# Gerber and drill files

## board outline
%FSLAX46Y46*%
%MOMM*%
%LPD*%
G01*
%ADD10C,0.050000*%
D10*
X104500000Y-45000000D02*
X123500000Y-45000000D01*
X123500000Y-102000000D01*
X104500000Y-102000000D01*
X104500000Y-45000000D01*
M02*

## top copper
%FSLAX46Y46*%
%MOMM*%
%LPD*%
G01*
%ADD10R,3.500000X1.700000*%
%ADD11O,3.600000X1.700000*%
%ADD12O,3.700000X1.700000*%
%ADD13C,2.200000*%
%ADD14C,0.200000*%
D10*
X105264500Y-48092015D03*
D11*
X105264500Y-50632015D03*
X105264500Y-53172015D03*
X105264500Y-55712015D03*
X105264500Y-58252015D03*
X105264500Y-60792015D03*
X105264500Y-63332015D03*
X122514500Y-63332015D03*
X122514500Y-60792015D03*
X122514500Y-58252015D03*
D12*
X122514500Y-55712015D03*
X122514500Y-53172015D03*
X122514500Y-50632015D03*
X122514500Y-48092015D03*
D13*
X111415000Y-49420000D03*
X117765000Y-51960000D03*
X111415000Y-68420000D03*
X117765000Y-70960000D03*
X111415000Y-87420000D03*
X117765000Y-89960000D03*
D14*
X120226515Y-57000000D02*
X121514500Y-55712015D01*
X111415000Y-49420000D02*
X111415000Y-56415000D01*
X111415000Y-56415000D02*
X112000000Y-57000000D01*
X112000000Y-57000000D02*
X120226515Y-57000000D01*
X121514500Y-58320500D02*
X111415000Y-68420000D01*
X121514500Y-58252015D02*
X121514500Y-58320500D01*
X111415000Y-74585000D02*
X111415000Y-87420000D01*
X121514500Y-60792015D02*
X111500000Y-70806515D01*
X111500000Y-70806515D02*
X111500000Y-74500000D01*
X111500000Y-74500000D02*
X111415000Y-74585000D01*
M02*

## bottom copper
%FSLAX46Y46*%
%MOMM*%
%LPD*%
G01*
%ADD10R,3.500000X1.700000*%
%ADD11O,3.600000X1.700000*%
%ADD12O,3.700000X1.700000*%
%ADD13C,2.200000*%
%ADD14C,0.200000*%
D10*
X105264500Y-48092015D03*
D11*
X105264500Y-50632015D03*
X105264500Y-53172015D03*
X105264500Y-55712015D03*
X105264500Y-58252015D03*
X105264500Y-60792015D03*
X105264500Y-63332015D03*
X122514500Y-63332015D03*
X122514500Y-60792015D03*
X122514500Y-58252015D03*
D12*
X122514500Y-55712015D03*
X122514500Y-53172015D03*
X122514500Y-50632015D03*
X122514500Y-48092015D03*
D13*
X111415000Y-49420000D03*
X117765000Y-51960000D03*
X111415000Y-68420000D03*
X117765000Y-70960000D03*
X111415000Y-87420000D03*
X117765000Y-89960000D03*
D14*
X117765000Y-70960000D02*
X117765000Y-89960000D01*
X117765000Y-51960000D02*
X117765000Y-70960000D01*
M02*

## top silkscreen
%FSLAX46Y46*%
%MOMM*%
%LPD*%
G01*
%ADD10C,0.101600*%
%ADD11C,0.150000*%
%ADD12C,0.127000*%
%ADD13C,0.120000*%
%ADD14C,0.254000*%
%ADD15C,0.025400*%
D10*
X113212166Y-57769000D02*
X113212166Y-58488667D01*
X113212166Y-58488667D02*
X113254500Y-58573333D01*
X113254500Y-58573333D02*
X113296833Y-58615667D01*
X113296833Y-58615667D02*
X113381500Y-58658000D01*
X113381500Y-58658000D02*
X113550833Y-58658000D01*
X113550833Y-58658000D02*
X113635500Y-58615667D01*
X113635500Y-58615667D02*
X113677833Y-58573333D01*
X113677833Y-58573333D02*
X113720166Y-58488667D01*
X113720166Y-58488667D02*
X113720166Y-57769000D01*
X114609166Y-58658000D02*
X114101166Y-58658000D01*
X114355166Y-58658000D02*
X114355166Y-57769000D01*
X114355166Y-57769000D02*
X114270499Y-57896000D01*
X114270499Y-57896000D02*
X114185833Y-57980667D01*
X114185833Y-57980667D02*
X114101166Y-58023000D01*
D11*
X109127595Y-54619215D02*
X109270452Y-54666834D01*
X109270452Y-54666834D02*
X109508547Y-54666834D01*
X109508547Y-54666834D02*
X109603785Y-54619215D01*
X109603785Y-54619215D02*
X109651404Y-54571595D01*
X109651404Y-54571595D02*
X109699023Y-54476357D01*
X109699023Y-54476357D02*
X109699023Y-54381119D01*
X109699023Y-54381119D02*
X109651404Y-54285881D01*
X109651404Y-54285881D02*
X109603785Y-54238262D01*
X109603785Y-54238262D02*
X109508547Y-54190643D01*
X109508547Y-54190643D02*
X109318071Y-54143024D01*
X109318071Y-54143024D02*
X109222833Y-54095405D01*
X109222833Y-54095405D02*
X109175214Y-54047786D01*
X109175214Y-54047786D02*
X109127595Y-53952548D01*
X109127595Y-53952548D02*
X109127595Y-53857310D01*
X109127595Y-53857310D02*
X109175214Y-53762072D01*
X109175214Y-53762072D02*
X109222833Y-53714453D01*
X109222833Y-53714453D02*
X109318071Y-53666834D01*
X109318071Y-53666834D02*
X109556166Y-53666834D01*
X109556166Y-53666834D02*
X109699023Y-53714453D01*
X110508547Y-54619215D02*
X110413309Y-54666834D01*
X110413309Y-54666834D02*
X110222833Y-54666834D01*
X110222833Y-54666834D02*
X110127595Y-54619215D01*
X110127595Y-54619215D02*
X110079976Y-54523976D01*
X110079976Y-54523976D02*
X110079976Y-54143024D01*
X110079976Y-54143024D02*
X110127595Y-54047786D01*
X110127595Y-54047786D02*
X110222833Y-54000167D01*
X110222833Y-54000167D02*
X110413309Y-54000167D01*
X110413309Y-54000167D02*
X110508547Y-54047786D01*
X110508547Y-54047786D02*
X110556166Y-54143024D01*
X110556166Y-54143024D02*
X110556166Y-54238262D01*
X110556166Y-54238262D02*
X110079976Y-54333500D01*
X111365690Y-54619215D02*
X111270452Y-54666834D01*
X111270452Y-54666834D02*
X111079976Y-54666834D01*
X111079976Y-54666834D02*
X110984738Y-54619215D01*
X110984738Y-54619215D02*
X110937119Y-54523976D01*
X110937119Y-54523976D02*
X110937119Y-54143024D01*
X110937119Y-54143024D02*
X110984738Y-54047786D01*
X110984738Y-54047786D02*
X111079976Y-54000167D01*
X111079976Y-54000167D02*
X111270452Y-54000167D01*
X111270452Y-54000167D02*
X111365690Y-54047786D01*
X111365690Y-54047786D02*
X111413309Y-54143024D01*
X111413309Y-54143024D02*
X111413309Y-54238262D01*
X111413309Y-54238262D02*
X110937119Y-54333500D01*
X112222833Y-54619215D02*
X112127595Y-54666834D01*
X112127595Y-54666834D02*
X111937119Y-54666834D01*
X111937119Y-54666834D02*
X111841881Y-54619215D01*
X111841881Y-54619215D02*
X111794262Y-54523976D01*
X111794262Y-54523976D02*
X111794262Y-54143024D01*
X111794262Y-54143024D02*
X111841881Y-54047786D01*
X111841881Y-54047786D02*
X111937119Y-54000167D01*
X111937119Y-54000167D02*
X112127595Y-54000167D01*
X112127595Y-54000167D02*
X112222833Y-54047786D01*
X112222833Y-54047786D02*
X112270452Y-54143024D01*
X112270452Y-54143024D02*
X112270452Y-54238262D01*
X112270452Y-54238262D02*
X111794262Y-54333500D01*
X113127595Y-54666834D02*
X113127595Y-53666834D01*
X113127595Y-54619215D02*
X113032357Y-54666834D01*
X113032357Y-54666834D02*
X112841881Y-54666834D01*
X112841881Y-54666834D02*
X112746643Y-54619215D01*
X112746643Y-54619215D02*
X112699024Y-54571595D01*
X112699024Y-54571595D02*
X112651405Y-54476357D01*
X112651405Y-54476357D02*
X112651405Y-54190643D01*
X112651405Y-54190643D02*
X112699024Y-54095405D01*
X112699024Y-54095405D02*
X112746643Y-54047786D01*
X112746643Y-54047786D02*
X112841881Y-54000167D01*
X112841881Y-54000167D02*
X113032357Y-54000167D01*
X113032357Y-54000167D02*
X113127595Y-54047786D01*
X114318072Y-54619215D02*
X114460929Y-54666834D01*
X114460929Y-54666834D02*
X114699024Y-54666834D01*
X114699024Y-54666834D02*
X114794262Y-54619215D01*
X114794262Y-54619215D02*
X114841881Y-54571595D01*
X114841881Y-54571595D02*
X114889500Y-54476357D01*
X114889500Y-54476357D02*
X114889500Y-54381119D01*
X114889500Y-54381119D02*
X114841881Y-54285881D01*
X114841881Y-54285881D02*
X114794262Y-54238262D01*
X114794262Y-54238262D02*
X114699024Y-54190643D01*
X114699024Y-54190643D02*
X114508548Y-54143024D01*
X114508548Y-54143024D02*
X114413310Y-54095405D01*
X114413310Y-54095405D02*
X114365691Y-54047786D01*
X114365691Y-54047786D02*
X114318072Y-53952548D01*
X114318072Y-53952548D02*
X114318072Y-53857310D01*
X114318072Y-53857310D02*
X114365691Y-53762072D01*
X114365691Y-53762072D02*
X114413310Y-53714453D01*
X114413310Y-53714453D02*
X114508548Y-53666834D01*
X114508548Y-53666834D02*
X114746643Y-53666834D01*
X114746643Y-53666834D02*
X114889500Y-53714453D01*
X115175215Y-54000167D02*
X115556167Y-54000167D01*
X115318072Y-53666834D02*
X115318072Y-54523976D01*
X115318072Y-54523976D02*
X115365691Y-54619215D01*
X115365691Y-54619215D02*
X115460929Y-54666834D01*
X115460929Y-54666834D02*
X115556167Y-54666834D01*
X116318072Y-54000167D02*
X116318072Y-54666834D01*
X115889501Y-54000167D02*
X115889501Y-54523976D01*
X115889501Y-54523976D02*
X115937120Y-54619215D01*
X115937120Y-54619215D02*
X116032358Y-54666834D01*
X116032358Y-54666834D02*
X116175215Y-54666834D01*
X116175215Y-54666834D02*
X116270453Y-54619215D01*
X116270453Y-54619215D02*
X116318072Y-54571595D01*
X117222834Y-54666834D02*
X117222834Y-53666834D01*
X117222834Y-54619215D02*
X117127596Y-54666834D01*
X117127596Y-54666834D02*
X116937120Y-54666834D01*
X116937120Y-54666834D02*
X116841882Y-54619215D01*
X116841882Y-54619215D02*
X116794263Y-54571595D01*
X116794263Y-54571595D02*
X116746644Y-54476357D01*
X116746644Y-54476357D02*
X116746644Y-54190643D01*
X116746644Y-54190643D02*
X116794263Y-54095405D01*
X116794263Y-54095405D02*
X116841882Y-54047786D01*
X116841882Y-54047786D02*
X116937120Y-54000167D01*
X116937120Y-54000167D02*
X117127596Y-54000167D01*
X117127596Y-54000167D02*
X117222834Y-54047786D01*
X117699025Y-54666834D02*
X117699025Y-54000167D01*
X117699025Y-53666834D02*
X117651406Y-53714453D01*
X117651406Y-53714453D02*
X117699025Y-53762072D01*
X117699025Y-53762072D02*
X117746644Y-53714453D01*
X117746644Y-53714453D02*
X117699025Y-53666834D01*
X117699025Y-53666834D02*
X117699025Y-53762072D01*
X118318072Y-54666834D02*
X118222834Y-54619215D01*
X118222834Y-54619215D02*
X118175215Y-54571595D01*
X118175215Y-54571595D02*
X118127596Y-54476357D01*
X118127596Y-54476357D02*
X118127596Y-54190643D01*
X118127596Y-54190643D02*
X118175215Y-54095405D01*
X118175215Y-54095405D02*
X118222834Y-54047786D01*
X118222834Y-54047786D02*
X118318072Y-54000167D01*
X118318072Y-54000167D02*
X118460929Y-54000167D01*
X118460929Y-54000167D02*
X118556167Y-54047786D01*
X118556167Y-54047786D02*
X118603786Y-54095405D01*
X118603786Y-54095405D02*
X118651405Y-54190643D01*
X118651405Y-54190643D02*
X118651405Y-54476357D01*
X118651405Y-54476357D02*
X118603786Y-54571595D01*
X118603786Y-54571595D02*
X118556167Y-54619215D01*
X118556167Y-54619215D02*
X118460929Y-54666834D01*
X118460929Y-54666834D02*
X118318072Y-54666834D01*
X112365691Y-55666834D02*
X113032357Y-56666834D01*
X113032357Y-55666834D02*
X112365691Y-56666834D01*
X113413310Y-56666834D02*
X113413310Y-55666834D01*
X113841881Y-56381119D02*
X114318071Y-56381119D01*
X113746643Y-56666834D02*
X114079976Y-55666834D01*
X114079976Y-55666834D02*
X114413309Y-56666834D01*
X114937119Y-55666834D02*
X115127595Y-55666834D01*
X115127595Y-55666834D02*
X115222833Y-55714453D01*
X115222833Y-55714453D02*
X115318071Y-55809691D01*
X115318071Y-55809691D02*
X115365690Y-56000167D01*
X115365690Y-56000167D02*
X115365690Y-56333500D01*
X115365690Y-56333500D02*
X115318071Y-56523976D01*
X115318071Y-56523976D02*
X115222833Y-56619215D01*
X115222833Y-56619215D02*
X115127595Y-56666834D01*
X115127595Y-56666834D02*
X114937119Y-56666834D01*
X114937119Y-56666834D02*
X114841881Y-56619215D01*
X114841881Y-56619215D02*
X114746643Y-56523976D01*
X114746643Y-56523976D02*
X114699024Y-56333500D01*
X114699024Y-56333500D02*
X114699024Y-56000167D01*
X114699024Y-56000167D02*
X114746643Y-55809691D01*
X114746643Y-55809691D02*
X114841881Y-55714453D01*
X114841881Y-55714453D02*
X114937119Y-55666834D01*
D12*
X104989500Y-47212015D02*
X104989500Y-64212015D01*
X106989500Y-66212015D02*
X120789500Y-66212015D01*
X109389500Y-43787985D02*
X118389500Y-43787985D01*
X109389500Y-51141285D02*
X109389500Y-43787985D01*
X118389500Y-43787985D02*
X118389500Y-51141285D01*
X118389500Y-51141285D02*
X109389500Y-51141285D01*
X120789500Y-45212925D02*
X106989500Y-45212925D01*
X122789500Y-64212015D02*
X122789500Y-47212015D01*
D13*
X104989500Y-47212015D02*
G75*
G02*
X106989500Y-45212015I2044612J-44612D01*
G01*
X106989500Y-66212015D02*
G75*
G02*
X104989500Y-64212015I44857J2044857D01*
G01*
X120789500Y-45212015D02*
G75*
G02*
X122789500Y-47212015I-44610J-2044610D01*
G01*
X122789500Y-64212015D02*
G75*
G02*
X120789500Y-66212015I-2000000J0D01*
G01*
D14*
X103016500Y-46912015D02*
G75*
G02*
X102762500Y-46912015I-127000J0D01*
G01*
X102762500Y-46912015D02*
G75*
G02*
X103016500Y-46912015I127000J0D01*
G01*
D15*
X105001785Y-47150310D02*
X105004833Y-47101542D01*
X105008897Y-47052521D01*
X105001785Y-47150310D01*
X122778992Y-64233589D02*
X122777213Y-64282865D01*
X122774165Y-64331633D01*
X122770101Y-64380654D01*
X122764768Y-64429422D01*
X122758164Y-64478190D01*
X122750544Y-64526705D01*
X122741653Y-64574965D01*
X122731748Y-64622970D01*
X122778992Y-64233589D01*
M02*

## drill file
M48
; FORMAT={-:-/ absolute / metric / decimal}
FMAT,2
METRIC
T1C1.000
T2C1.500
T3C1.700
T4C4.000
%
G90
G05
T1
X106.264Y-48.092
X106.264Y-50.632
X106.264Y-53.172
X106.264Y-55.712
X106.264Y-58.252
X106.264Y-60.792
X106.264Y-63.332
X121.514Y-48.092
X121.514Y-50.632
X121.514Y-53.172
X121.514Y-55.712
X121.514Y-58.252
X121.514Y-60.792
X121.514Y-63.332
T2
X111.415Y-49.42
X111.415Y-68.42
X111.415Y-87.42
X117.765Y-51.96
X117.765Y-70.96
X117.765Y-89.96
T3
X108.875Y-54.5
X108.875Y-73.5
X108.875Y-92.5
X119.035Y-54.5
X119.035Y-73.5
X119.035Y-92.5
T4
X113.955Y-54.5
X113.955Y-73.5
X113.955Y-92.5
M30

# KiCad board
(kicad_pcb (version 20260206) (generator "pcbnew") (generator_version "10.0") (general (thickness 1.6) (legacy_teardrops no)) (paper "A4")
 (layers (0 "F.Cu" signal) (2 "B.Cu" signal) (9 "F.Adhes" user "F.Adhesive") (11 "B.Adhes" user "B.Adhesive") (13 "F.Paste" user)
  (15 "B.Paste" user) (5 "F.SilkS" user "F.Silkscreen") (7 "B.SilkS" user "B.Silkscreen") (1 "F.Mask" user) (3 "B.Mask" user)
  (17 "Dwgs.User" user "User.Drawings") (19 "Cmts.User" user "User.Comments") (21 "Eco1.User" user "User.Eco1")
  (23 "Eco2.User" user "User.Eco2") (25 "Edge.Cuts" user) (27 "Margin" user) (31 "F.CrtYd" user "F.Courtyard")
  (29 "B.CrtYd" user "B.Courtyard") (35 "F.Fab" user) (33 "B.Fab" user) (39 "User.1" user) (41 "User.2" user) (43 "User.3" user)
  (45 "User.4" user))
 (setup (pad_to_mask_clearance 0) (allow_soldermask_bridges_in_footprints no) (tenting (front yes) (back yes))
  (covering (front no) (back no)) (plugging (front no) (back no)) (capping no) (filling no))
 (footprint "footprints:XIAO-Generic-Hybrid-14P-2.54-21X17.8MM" (layer "F.Cu") (at 113.8895 55.712015)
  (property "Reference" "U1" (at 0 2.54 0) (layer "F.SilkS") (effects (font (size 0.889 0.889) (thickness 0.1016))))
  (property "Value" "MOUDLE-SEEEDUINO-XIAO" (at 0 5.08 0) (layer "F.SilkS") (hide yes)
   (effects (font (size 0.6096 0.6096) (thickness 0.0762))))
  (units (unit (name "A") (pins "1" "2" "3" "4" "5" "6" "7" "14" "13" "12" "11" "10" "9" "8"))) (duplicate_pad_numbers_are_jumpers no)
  (fp_line (start -8.9 -8.5) (end -8.9 8.5) (stroke (width 0.127) (type solid)) (layer "F.SilkS"))
  (fp_line (start -6.9 10.5) (end 6.9 10.5) (stroke (width 0.127) (type solid)) (layer "F.SilkS"))
  (fp_line (start -4.5 -11.92403) (end 4.5 -11.92403) (stroke (width 0.127) (type solid)) (layer "F.SilkS"))
  (fp_line (start -4.5 -4.57073) (end -4.5 -11.92403) (stroke (width 0.127) (type solid)) (layer "F.SilkS"))
  (fp_line (start 4.5 -11.92403) (end 4.5 -4.57073) (stroke (width 0.127) (type solid)) (layer "F.SilkS"))
  (fp_line (start 4.5 -4.57073) (end -4.5 -4.57073) (stroke (width 0.127) (type solid)) (layer "F.SilkS"))
  (fp_line (start 6.9 -10.49909) (end -6.9 -10.49909) (stroke (width 0.127) (type solid)) (layer "F.SilkS"))
  (fp_line (start 8.9 8.5) (end 8.9 -8.5) (stroke (width 0.127) (type solid)) (layer "F.SilkS"))
  (fp_arc (start -8.9 -8.5) (mid -8.301491 -9.901491) (end -6.9 -10.5) (stroke (width 0.12) (type solid)) (layer "F.SilkS"))
  (fp_arc (start -6.9 10.5) (mid -8.301423 9.901423) (end -8.9 8.5) (stroke (width 0.12) (type solid)) (layer "F.SilkS"))
  (fp_arc (start 6.9 -10.5) (mid 8.301491 -9.901491) (end 8.9 -8.5) (stroke (width 0.12) (type solid)) (layer "F.SilkS"))
  (fp_arc (start 8.9 8.5) (mid 8.314214 9.914214) (end 6.9 10.5) (stroke (width 0.12) (type solid)) (layer "F.SilkS"))
  (fp_circle (center -11 -8.8) (end -11 -9.054) (stroke (width 0) (type solid)) (fill yes) (layer "F.SilkS"))
  (fp_poly
   (pts (xy -8.887715 -8.561705) (xy -8.884667 -8.610473) (xy -8.880603 -8.659494)) (stroke (width 0.0254) (type solid)) (fill no)
   (layer "F.SilkS"))
  (fp_poly
   (pts (xy 8.889492 8.521574) (xy 8.887713 8.57085) (xy 8.884665 8.619618) (xy 8.880601 8.668639) (xy 8.875268 8.717407)
    (xy 8.868664 8.766175) (xy 8.861044 8.81469) (xy 8.852153 8.86295) (xy 8.842248 8.910955))
   (stroke (width 0.0254) (type solid)) (fill no) (layer "F.SilkS"))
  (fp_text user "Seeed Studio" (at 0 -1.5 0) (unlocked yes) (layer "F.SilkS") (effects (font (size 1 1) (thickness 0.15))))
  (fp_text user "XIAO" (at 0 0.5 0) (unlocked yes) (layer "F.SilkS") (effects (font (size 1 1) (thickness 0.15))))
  (pad "1" thru_hole rect (at -7.625 -7.62) (size 3.5 1.7) (drill 1 (offset -1 0)) (layers "*.Cu" "*.Mask") (remove_unused_layers no)
   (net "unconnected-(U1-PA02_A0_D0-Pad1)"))
  (pad "2" thru_hole oval (at -7.625 -5.08) (size 3.6 1.7) (drill 1 (offset -1 0)) (layers "*.Cu" "*.Mask") (remove_unused_layers no)
   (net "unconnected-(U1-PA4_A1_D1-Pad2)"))
  (pad "3" thru_hole oval (at -7.625 -2.54) (size 3.6 1.7) (drill 1 (offset -1 0)) (layers "*.Cu" "*.Mask") (remove_unused_layers no)
   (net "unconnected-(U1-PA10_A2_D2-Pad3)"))
  (pad "4" thru_hole oval (at -7.625 0) (size 3.6 1.7) (drill 1 (offset -1 0)) (layers "*.Cu" "*.Mask") (remove_unused_layers no)
   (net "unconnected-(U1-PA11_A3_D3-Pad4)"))
  (pad "5" thru_hole oval (at -7.625 2.54) (size 3.6 1.7) (drill 1 (offset -1 0)) (layers "*.Cu" "*.Mask") (remove_unused_layers no)
   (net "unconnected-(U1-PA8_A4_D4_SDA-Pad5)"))
  (pad "6" thru_hole oval (at -7.625 5.08 180) (size 3.6 1.7) (drill 1 (offset 1 0)) (layers "*.Cu" "*.Mask") (remove_unused_layers no)
   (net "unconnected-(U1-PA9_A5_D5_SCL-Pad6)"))
  (pad "7" thru_hole oval (at -7.625 7.62) (size 3.6 1.7) (drill 1 (offset -1 0)) (layers "*.Cu" "*.Mask") (remove_unused_layers no)
   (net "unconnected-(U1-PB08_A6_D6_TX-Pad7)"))
  (pad "8" thru_hole oval (at 7.625 7.62) (size 3.6 1.7) (drill 1 (offset 1 0)) (layers "*.Cu" "*.Mask") (remove_unused_layers no)
   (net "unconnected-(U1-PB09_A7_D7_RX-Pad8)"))
  (pad "9" thru_hole oval (at 7.625 5.08) (size 3.6 1.7) (drill 1 (offset 1 0)) (layers "*.Cu" "*.Mask") (remove_unused_layers no)
   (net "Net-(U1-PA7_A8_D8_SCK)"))
  (pad "10" thru_hole oval (at 7.625 2.54) (size 3.6 1.7) (drill 1 (offset 1 0)) (layers "*.Cu" "*.Mask") (remove_unused_layers no)
   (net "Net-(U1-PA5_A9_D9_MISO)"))
  (pad "11" thru_hole oval (at 7.625 0) (size 3.7 1.7) (drill 1 (offset 1 0)) (layers "*.Cu" "*.Mask") (remove_unused_layers no)
   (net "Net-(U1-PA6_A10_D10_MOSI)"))
  (pad "12" thru_hole oval (at 7.625 -2.54) (size 3.7 1.7) (drill 1 (offset 1 0)) (layers "*.Cu" "*.Mask") (remove_unused_layers no)
   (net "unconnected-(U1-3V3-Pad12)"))
  (pad "13" thru_hole oval (at 7.625 -5.08) (size 3.7 1.7) (drill 1 (offset 1 0)) (layers "*.Cu" "*.Mask") (remove_unused_layers no)
   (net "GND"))
  (pad "14" thru_hole oval (at 7.625 -7.62) (size 3.7 1.7) (drill 1 (offset 1 0)) (layers "*.Cu" "*.Mask") (remove_unused_layers no)
   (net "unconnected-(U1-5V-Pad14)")))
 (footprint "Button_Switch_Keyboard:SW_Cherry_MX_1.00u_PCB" (layer "B.Cu") (at 111.415 49.42 180)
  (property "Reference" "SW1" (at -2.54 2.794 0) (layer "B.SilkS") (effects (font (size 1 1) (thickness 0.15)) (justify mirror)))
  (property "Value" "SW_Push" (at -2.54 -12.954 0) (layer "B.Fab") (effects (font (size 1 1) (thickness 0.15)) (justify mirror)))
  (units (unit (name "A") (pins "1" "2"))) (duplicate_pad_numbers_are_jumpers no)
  (pad "" np_thru_hole circle (at -7.62 -5.08 180) (size 1.7 1.7) (drill 1.7) (layers "*.Cu" "*.Mask"))
  (pad "" np_thru_hole circle (at -2.54 -5.08 180) (size 4 4) (drill 4) (layers "*.Cu" "*.Mask"))
  (pad "" np_thru_hole circle (at 2.54 -5.08 180) (size 1.7 1.7) (drill 1.7) (layers "*.Cu" "*.Mask"))
  (pad "1" thru_hole circle (at 0 0 180) (size 2.2 2.2) (drill 1.5) (layers "*.Cu" "*.Mask") (remove_unused_layers no)
   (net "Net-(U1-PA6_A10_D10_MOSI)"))
  (pad "2" thru_hole circle (at -6.35 -2.54 180) (size 2.2 2.2) (drill 1.5) (layers "*.Cu" "*.Mask") (remove_unused_layers no) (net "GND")))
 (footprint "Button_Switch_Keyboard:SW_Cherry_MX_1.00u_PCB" (layer "B.Cu") (at 111.415 68.42 180)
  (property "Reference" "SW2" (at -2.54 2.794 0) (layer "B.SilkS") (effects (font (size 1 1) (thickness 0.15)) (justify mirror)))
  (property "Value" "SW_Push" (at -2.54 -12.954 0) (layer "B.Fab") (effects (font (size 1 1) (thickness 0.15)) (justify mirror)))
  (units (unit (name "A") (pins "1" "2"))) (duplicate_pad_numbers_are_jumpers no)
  (pad "" np_thru_hole circle (at -7.62 -5.08 180) (size 1.7 1.7) (drill 1.7) (layers "*.Cu" "*.Mask"))
  (pad "" np_thru_hole circle (at -2.54 -5.08 180) (size 4 4) (drill 4) (layers "*.Cu" "*.Mask"))
  (pad "" np_thru_hole circle (at 2.54 -5.08 180) (size 1.7 1.7) (drill 1.7) (layers "*.Cu" "*.Mask"))
  (pad "1" thru_hole circle (at 0 0 180) (size 2.2 2.2) (drill 1.5) (layers "*.Cu" "*.Mask") (remove_unused_layers no)
   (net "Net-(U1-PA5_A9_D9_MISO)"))
  (pad "2" thru_hole circle (at -6.35 -2.54 180) (size 2.2 2.2) (drill 1.5) (layers "*.Cu" "*.Mask") (remove_unused_layers no) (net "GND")))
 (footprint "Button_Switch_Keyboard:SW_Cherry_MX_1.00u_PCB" (layer "B.Cu") (at 111.415 87.42 180)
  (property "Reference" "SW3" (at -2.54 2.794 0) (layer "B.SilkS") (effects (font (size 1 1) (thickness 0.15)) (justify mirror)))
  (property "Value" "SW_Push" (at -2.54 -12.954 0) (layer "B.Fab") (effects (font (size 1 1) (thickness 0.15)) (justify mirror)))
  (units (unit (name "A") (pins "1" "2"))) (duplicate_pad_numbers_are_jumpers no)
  (pad "" np_thru_hole circle (at -7.62 -5.08 180) (size 1.7 1.7) (drill 1.7) (layers "*.Cu" "*.Mask"))
  (pad "" np_thru_hole circle (at -2.54 -5.08 180) (size 4 4) (drill 4) (layers "*.Cu" "*.Mask"))
  (pad "" np_thru_hole circle (at 2.54 -5.08 180) (size 1.7 1.7) (drill 1.7) (layers "*.Cu" "*.Mask"))
  (pad "1" thru_hole circle (at 0 0 180) (size 2.2 2.2) (drill 1.5) (layers "*.Cu" "*.Mask") (remove_unused_layers no)
   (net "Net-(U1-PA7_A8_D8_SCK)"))
  (pad "2" thru_hole circle (at -6.35 -2.54 180) (size 2.2 2.2) (drill 1.5) (layers "*.Cu" "*.Mask") (remove_unused_layers no) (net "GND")))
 (gr_rect (start 104.5 45) (end 123.5 102) (stroke (width 0.05) (type default)) (fill no) (layer "Edge.Cuts"))
 (segment (start 120.226515 57) (end 121.5145 55.712015) (width 0.2) (layer "F.Cu") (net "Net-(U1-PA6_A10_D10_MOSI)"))
 (segment (start 111.415 49.42) (end 111.415 56.415) (width 0.2) (layer "F.Cu") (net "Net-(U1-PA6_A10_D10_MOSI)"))
 (segment (start 111.415 56.415) (end 112 57) (width 0.2) (layer "F.Cu") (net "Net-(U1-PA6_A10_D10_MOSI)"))
 (segment (start 112 57) (end 120.226515 57) (width 0.2) (layer "F.Cu") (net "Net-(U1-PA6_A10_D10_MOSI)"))
 (segment (start 117.765 70.96) (end 117.765 89.96) (width 0.2) (layer "B.Cu") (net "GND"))
 (segment (start 117.765 51.96) (end 117.765 70.96) (width 0.2) (layer "B.Cu") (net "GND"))
 (segment (start 121.5145 58.3205) (end 111.415 68.42) (width 0.2) (layer "F.Cu") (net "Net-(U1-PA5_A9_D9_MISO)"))
 (segment (start 121.5145 58.252015) (end 121.5145 58.3205) (width 0.2) (layer "F.Cu") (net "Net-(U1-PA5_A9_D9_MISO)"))
 (segment (start 111.415 74.585) (end 111.415 87.42) (width 0.2) (layer "F.Cu") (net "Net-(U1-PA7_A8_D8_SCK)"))
 (segment (start 121.5145 60.792015) (end 111.5 70.806515) (width 0.2) (layer "F.Cu") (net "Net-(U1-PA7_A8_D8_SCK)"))
 (segment (start 111.5 70.806515) (end 111.5 74.5) (width 0.2) (layer "F.Cu") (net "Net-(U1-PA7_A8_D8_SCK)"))
 (segment (start 111.5 74.5) (end 111.415 74.585) (width 0.2) (layer "F.Cu") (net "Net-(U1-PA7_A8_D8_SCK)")))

